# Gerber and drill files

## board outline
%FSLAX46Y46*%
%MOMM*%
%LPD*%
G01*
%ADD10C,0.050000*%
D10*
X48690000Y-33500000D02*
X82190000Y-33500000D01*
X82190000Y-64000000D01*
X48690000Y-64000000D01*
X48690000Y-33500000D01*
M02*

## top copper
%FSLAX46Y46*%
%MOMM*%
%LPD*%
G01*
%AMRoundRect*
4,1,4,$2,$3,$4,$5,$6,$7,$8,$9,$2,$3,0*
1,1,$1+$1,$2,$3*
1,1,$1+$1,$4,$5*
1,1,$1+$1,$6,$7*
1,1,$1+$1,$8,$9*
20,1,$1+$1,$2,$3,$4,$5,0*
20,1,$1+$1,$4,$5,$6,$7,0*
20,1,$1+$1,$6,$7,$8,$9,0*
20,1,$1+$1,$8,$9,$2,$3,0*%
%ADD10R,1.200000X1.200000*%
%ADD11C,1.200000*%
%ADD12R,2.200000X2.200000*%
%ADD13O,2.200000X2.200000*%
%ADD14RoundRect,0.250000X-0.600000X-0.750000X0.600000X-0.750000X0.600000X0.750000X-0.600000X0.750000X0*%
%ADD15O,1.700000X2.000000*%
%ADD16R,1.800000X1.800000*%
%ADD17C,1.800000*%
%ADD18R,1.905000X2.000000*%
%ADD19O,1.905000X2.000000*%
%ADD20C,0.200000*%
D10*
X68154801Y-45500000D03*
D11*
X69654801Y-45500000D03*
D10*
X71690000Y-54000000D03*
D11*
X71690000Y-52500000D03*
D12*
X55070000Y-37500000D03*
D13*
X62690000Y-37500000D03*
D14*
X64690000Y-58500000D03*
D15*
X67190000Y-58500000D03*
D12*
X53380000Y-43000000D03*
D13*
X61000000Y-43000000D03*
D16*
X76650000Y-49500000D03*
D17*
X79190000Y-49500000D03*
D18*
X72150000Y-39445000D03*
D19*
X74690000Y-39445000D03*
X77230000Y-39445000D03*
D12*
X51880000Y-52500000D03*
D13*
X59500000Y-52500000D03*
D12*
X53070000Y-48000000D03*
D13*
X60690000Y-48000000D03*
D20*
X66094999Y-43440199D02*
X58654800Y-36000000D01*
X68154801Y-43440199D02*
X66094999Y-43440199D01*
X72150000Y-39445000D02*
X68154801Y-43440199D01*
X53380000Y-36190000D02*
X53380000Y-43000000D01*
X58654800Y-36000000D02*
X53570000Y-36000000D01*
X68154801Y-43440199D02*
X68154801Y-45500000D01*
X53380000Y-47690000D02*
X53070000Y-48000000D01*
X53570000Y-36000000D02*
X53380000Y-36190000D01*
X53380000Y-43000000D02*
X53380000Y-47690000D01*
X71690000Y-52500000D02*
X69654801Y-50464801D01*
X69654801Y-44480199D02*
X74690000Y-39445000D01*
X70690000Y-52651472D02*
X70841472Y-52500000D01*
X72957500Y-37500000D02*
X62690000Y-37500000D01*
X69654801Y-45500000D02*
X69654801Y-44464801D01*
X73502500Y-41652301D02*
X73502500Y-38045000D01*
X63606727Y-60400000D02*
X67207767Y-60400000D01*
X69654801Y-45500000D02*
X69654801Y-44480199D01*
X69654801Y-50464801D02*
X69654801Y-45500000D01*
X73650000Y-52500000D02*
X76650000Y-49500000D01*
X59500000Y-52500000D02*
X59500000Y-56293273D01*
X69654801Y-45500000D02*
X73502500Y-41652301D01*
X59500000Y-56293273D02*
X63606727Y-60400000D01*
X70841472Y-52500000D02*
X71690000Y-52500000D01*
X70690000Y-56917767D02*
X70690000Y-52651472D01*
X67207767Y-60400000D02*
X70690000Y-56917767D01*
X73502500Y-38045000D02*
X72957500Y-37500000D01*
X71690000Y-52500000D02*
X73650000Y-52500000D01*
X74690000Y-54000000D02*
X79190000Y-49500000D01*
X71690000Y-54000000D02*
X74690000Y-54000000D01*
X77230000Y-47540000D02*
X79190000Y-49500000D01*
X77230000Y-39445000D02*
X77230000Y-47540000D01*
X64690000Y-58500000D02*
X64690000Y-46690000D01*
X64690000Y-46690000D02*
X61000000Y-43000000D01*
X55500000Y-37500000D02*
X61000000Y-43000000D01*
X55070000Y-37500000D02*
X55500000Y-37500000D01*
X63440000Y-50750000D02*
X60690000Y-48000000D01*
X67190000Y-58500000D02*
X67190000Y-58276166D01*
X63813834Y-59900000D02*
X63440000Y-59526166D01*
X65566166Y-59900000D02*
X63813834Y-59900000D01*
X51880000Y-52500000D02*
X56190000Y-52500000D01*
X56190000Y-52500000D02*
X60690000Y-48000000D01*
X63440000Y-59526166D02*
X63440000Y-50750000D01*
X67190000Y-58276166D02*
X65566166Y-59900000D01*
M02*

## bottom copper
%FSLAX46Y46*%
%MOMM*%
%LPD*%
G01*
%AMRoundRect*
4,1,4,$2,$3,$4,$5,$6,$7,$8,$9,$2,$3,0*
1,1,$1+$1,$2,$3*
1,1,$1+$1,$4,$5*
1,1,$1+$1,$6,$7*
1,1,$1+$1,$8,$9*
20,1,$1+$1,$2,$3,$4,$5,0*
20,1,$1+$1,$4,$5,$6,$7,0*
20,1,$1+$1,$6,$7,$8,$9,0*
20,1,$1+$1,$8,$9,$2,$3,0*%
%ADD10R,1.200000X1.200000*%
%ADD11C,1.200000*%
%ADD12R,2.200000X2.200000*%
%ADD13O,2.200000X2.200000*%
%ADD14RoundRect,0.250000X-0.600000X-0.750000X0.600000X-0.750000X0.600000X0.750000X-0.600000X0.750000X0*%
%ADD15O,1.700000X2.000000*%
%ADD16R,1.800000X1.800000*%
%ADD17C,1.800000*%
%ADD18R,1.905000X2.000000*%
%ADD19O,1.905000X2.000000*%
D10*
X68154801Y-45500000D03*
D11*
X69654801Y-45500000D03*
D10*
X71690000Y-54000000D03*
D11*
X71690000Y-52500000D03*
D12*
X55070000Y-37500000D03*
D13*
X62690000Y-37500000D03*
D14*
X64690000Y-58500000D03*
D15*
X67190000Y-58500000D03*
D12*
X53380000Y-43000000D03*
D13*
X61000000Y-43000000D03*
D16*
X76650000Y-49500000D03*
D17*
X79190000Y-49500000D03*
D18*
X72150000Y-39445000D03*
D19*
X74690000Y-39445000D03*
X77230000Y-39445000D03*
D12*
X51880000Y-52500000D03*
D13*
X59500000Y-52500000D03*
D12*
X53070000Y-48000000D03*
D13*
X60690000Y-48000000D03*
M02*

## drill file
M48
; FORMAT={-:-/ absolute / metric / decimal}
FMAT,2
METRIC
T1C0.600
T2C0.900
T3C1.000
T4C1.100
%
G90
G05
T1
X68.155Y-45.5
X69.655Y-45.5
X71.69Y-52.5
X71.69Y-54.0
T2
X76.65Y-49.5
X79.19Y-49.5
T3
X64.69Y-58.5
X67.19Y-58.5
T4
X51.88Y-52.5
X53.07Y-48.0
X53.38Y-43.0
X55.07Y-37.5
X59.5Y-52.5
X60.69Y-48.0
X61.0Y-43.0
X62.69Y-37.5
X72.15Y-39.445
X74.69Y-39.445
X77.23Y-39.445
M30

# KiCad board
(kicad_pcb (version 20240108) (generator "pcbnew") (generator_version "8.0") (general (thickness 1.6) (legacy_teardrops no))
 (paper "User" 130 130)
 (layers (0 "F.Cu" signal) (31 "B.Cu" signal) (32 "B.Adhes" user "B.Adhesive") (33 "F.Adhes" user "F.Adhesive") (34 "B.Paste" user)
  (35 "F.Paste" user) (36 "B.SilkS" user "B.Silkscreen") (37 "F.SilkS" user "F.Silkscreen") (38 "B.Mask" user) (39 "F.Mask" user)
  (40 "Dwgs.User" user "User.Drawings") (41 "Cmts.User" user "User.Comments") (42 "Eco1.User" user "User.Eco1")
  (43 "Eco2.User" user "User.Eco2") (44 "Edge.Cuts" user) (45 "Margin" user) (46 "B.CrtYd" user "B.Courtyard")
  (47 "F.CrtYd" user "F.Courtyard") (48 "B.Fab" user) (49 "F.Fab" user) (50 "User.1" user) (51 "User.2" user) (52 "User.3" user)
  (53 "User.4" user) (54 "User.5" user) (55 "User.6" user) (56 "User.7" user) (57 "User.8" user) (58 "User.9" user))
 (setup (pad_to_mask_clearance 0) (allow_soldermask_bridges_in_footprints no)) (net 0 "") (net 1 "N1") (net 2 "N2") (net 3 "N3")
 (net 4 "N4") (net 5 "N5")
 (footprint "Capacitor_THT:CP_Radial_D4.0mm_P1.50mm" (layer "F.Cu") (at 68.154801 45.5)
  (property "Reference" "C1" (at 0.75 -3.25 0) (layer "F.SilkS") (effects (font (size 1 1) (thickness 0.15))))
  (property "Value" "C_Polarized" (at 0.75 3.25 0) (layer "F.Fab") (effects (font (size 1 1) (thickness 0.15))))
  (pad "1" thru_hole rect (at 0 0) (size 1.2 1.2) (drill 0.6) (layers "*.Cu" "*.Mask") (remove_unused_layers no) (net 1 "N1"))
  (pad "2" thru_hole circle (at 1.5 0) (size 1.2 1.2) (drill 0.6) (layers "*.Cu" "*.Mask") (remove_unused_layers no) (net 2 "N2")))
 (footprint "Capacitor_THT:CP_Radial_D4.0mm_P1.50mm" (layer "F.Cu") (at 71.69 54 90)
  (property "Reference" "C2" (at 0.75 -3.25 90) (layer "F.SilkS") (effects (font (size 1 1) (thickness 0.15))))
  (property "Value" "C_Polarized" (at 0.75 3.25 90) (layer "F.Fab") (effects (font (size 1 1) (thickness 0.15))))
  (pad "1" thru_hole rect (at 0 0 90) (size 1.2 1.2) (drill 0.6) (layers "*.Cu" "*.Mask") (remove_unused_layers no) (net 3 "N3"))
  (pad "2" thru_hole circle (at 1.5 0 90) (size 1.2 1.2) (drill 0.6) (layers "*.Cu" "*.Mask") (remove_unused_layers no) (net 2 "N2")))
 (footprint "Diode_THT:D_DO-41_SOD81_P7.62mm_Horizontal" (layer "F.Cu") (at 55.07 37.5)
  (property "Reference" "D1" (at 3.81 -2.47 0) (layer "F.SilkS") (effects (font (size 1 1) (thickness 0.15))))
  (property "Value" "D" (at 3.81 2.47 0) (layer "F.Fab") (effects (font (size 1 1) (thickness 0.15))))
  (pad "1" thru_hole rect (at 0 0) (size 2.2 2.2) (drill 1.1) (layers "*.Cu" "*.Mask") (remove_unused_layers no) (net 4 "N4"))
  (pad "2" thru_hole oval (at 7.62 0) (size 2.2 2.2) (drill 1.1) (layers "*.Cu" "*.Mask") (remove_unused_layers no) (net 2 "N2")))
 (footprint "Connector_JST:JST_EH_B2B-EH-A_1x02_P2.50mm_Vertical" (layer "F.Cu") (at 64.69 58.5)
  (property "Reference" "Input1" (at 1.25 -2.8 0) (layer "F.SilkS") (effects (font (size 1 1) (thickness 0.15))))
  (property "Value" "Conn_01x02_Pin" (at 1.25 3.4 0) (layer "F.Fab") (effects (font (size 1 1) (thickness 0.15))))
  (pad "1" thru_hole roundrect (at 0 0) (size 1.7 2) (drill 1) (layers "*.Cu" "*.Mask") (remove_unused_layers no)
   (roundrect_rratio 0.147059) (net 4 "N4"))
  (pad "2" thru_hole oval (at 2.5 0) (size 1.7 2) (drill 1) (layers "*.Cu" "*.Mask") (remove_unused_layers no) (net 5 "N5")))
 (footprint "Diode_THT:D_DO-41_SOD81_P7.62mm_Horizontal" (layer "F.Cu") (at 53.38 43)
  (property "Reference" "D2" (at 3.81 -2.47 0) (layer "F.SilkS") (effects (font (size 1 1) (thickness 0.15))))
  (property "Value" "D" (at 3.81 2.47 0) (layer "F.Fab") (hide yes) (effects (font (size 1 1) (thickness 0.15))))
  (pad "1" thru_hole rect (at 0 0) (size 2.2 2.2) (drill 1.1) (layers "*.Cu" "*.Mask") (remove_unused_layers no) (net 1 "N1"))
  (pad "2" thru_hole oval (at 7.62 0) (size 2.2 2.2) (drill 1.1) (layers "*.Cu" "*.Mask") (remove_unused_layers no) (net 4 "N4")))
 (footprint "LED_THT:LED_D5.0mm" (layer "F.Cu") (at 76.65 49.5)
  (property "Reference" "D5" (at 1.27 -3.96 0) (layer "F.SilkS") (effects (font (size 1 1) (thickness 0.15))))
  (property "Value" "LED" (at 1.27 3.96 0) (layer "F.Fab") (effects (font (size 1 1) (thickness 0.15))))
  (pad "1" thru_hole rect (at 0 0) (size 1.8 1.8) (drill 0.9) (layers "*.Cu" "*.Mask") (remove_unused_layers no) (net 2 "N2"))
  (pad "2" thru_hole circle (at 2.54 0) (size 1.8 1.8) (drill 0.9) (layers "*.Cu" "*.Mask") (remove_unused_layers no) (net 3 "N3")))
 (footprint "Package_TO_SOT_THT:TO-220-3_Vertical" (layer "F.Cu") (at 72.15 39.445)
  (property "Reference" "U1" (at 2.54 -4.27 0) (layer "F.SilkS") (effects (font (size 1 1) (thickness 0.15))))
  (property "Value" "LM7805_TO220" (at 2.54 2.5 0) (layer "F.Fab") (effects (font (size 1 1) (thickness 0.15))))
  (pad "1" thru_hole rect (at 0 0) (size 1.905 2) (drill 1.1) (layers "*.Cu" "*.Mask") (remove_unused_layers no) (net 1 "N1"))
  (pad "2" thru_hole oval (at 2.54 0) (size 1.905 2) (drill 1.1) (layers "*.Cu" "*.Mask") (remove_unused_layers no) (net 2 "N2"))
  (pad "3" thru_hole oval (at 5.08 0) (size 1.905 2) (drill 1.1) (layers "*.Cu" "*.Mask") (remove_unused_layers no) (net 3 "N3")))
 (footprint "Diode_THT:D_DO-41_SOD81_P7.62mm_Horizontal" (layer "F.Cu") (at 51.88 52.5)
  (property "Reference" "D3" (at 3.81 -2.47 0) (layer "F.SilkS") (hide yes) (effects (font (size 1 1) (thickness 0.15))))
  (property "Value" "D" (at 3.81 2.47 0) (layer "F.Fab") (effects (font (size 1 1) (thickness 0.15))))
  (pad "1" thru_hole rect (at 0 0) (size 2.2 2.2) (drill 1.1) (layers "*.Cu" "*.Mask") (remove_unused_layers no) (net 5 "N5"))
  (pad "2" thru_hole oval (at 7.62 0) (size 2.2 2.2) (drill 1.1) (layers "*.Cu" "*.Mask") (remove_unused_layers no) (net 2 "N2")))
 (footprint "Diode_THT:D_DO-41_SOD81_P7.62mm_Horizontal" (layer "F.Cu") (at 53.07 48)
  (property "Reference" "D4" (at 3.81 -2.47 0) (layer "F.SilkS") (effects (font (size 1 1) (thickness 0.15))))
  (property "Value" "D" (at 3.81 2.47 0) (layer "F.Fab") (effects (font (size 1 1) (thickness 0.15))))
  (pad "1" thru_hole rect (at 0 0) (size 2.2 2.2) (drill 1.1) (layers "*.Cu" "*.Mask") (remove_unused_layers no) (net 1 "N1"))
  (pad "2" thru_hole oval (at 7.62 0) (size 2.2 2.2) (drill 1.1) (layers "*.Cu" "*.Mask") (remove_unused_layers no) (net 5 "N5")))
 (gr_rect (start 48.69 33.5) (end 82.19 64) (stroke (width 0.05) (type default)) (fill none) (layer "Edge.Cuts"))
 (segment (start 66.094999 43.440199) (end 58.6548 36) (width 0.2) (layer "F.Cu") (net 1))
 (segment (start 68.154801 43.440199) (end 66.094999 43.440199) (width 0.2) (layer "F.Cu") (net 1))
 (segment (start 72.15 39.445) (end 68.154801 43.440199) (width 0.2) (layer "F.Cu") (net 1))
 (segment (start 53.38 36.19) (end 53.38 43) (width 0.2) (layer "F.Cu") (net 1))
 (segment (start 58.6548 36) (end 53.57 36) (width 0.2) (layer "F.Cu") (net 1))
 (segment (start 68.154801 43.440199) (end 68.154801 45.5) (width 0.2) (layer "F.Cu") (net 1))
 (segment (start 53.38 47.69) (end 53.07 48) (width 0.2) (layer "F.Cu") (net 1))
 (segment (start 53.57 36) (end 53.38 36.19) (width 0.2) (layer "F.Cu") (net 1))
 (segment (start 53.38 43) (end 53.38 47.69) (width 0.2) (layer "F.Cu") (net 1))
 (segment (start 71.69 52.5) (end 69.654801 50.464801) (width 0.2) (layer "F.Cu") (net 2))
 (segment (start 69.654801 44.480199) (end 74.69 39.445) (width 0.2) (layer "F.Cu") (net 2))
 (segment (start 70.69 52.651472) (end 70.841472 52.5) (width 0.2) (layer "F.Cu") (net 2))
 (segment (start 72.9575 37.5) (end 62.69 37.5) (width 0.2) (layer "F.Cu") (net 2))
 (segment (start 69.654801 45.5) (end 69.654801 44.464801) (width 0.2) (layer "F.Cu") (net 2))
 (segment (start 73.5025 41.652301) (end 73.5025 38.045) (width 0.2) (layer "F.Cu") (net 2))
 (segment (start 63.606727 60.4) (end 67.207767 60.4) (width 0.2) (layer "F.Cu") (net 2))
 (segment (start 69.654801 45.5) (end 69.654801 44.480199) (width 0.2) (layer "F.Cu") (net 2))
 (segment (start 69.654801 50.464801) (end 69.654801 45.5) (width 0.2) (layer "F.Cu") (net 2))
 (segment (start 73.65 52.5) (end 76.65 49.5) (width 0.2) (layer "F.Cu") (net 2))
 (segment (start 59.5 52.5) (end 59.5 56.293273) (width 0.2) (layer "F.Cu") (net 2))
 (segment (start 69.654801 45.5) (end 73.5025 41.652301) (width 0.2) (layer "F.Cu") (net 2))
 (segment (start 59.5 56.293273) (end 63.606727 60.4) (width 0.2) (layer "F.Cu") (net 2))
 (segment (start 70.841472 52.5) (end 71.69 52.5) (width 0.2) (layer "F.Cu") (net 2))
 (segment (start 70.69 56.917767) (end 70.69 52.651472) (width 0.2) (layer "F.Cu") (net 2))
 (segment (start 67.207767 60.4) (end 70.69 56.917767) (width 0.2) (layer "F.Cu") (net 2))
 (segment (start 73.5025 38.045) (end 72.9575 37.5) (width 0.2) (layer "F.Cu") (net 2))
 (segment (start 71.69 52.5) (end 73.65 52.5) (width 0.2) (layer "F.Cu") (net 2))
 (segment (start 74.69 54) (end 79.19 49.5) (width 0.2) (layer "F.Cu") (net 3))
 (segment (start 71.69 54) (end 74.69 54) (width 0.2) (layer "F.Cu") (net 3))
 (segment (start 77.23 47.54) (end 79.19 49.5) (width 0.2) (layer "F.Cu") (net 3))
 (segment (start 77.23 39.445) (end 77.23 47.54) (width 0.2) (layer "F.Cu") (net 3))
 (segment (start 64.69 58.5) (end 64.69 46.69) (width 0.2) (layer "F.Cu") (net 4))
 (segment (start 64.69 46.69) (end 61 43) (width 0.2) (layer "F.Cu") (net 4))
 (segment (start 55.5 37.5) (end 61 43) (width 0.2) (layer "F.Cu") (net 4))
 (segment (start 55.07 37.5) (end 55.5 37.5) (width 0.2) (layer "F.Cu") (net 4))
 (segment (start 63.44 50.75) (end 60.69 48) (width 0.2) (layer "F.Cu") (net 5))
 (segment (start 67.19 58.5) (end 67.19 58.276166) (width 0.2) (layer "F.Cu") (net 5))
 (segment (start 63.813834 59.9) (end 63.44 59.526166) (width 0.2) (layer "F.Cu") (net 5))
 (segment (start 65.566166 59.9) (end 63.813834 59.9) (width 0.2) (layer "F.Cu") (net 5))
 (segment (start 51.88 52.5) (end 56.19 52.5) (width 0.2) (layer "F.Cu") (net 5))
 (segment (start 56.19 52.5) (end 60.69 48) (width 0.2) (layer "F.Cu") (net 5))
 (segment (start 63.44 59.526166) (end 63.44 50.75) (width 0.2) (layer "F.Cu") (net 5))
 (segment (start 67.19 58.276166) (end 65.566166 59.9) (width 0.2) (layer "F.Cu") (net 5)))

